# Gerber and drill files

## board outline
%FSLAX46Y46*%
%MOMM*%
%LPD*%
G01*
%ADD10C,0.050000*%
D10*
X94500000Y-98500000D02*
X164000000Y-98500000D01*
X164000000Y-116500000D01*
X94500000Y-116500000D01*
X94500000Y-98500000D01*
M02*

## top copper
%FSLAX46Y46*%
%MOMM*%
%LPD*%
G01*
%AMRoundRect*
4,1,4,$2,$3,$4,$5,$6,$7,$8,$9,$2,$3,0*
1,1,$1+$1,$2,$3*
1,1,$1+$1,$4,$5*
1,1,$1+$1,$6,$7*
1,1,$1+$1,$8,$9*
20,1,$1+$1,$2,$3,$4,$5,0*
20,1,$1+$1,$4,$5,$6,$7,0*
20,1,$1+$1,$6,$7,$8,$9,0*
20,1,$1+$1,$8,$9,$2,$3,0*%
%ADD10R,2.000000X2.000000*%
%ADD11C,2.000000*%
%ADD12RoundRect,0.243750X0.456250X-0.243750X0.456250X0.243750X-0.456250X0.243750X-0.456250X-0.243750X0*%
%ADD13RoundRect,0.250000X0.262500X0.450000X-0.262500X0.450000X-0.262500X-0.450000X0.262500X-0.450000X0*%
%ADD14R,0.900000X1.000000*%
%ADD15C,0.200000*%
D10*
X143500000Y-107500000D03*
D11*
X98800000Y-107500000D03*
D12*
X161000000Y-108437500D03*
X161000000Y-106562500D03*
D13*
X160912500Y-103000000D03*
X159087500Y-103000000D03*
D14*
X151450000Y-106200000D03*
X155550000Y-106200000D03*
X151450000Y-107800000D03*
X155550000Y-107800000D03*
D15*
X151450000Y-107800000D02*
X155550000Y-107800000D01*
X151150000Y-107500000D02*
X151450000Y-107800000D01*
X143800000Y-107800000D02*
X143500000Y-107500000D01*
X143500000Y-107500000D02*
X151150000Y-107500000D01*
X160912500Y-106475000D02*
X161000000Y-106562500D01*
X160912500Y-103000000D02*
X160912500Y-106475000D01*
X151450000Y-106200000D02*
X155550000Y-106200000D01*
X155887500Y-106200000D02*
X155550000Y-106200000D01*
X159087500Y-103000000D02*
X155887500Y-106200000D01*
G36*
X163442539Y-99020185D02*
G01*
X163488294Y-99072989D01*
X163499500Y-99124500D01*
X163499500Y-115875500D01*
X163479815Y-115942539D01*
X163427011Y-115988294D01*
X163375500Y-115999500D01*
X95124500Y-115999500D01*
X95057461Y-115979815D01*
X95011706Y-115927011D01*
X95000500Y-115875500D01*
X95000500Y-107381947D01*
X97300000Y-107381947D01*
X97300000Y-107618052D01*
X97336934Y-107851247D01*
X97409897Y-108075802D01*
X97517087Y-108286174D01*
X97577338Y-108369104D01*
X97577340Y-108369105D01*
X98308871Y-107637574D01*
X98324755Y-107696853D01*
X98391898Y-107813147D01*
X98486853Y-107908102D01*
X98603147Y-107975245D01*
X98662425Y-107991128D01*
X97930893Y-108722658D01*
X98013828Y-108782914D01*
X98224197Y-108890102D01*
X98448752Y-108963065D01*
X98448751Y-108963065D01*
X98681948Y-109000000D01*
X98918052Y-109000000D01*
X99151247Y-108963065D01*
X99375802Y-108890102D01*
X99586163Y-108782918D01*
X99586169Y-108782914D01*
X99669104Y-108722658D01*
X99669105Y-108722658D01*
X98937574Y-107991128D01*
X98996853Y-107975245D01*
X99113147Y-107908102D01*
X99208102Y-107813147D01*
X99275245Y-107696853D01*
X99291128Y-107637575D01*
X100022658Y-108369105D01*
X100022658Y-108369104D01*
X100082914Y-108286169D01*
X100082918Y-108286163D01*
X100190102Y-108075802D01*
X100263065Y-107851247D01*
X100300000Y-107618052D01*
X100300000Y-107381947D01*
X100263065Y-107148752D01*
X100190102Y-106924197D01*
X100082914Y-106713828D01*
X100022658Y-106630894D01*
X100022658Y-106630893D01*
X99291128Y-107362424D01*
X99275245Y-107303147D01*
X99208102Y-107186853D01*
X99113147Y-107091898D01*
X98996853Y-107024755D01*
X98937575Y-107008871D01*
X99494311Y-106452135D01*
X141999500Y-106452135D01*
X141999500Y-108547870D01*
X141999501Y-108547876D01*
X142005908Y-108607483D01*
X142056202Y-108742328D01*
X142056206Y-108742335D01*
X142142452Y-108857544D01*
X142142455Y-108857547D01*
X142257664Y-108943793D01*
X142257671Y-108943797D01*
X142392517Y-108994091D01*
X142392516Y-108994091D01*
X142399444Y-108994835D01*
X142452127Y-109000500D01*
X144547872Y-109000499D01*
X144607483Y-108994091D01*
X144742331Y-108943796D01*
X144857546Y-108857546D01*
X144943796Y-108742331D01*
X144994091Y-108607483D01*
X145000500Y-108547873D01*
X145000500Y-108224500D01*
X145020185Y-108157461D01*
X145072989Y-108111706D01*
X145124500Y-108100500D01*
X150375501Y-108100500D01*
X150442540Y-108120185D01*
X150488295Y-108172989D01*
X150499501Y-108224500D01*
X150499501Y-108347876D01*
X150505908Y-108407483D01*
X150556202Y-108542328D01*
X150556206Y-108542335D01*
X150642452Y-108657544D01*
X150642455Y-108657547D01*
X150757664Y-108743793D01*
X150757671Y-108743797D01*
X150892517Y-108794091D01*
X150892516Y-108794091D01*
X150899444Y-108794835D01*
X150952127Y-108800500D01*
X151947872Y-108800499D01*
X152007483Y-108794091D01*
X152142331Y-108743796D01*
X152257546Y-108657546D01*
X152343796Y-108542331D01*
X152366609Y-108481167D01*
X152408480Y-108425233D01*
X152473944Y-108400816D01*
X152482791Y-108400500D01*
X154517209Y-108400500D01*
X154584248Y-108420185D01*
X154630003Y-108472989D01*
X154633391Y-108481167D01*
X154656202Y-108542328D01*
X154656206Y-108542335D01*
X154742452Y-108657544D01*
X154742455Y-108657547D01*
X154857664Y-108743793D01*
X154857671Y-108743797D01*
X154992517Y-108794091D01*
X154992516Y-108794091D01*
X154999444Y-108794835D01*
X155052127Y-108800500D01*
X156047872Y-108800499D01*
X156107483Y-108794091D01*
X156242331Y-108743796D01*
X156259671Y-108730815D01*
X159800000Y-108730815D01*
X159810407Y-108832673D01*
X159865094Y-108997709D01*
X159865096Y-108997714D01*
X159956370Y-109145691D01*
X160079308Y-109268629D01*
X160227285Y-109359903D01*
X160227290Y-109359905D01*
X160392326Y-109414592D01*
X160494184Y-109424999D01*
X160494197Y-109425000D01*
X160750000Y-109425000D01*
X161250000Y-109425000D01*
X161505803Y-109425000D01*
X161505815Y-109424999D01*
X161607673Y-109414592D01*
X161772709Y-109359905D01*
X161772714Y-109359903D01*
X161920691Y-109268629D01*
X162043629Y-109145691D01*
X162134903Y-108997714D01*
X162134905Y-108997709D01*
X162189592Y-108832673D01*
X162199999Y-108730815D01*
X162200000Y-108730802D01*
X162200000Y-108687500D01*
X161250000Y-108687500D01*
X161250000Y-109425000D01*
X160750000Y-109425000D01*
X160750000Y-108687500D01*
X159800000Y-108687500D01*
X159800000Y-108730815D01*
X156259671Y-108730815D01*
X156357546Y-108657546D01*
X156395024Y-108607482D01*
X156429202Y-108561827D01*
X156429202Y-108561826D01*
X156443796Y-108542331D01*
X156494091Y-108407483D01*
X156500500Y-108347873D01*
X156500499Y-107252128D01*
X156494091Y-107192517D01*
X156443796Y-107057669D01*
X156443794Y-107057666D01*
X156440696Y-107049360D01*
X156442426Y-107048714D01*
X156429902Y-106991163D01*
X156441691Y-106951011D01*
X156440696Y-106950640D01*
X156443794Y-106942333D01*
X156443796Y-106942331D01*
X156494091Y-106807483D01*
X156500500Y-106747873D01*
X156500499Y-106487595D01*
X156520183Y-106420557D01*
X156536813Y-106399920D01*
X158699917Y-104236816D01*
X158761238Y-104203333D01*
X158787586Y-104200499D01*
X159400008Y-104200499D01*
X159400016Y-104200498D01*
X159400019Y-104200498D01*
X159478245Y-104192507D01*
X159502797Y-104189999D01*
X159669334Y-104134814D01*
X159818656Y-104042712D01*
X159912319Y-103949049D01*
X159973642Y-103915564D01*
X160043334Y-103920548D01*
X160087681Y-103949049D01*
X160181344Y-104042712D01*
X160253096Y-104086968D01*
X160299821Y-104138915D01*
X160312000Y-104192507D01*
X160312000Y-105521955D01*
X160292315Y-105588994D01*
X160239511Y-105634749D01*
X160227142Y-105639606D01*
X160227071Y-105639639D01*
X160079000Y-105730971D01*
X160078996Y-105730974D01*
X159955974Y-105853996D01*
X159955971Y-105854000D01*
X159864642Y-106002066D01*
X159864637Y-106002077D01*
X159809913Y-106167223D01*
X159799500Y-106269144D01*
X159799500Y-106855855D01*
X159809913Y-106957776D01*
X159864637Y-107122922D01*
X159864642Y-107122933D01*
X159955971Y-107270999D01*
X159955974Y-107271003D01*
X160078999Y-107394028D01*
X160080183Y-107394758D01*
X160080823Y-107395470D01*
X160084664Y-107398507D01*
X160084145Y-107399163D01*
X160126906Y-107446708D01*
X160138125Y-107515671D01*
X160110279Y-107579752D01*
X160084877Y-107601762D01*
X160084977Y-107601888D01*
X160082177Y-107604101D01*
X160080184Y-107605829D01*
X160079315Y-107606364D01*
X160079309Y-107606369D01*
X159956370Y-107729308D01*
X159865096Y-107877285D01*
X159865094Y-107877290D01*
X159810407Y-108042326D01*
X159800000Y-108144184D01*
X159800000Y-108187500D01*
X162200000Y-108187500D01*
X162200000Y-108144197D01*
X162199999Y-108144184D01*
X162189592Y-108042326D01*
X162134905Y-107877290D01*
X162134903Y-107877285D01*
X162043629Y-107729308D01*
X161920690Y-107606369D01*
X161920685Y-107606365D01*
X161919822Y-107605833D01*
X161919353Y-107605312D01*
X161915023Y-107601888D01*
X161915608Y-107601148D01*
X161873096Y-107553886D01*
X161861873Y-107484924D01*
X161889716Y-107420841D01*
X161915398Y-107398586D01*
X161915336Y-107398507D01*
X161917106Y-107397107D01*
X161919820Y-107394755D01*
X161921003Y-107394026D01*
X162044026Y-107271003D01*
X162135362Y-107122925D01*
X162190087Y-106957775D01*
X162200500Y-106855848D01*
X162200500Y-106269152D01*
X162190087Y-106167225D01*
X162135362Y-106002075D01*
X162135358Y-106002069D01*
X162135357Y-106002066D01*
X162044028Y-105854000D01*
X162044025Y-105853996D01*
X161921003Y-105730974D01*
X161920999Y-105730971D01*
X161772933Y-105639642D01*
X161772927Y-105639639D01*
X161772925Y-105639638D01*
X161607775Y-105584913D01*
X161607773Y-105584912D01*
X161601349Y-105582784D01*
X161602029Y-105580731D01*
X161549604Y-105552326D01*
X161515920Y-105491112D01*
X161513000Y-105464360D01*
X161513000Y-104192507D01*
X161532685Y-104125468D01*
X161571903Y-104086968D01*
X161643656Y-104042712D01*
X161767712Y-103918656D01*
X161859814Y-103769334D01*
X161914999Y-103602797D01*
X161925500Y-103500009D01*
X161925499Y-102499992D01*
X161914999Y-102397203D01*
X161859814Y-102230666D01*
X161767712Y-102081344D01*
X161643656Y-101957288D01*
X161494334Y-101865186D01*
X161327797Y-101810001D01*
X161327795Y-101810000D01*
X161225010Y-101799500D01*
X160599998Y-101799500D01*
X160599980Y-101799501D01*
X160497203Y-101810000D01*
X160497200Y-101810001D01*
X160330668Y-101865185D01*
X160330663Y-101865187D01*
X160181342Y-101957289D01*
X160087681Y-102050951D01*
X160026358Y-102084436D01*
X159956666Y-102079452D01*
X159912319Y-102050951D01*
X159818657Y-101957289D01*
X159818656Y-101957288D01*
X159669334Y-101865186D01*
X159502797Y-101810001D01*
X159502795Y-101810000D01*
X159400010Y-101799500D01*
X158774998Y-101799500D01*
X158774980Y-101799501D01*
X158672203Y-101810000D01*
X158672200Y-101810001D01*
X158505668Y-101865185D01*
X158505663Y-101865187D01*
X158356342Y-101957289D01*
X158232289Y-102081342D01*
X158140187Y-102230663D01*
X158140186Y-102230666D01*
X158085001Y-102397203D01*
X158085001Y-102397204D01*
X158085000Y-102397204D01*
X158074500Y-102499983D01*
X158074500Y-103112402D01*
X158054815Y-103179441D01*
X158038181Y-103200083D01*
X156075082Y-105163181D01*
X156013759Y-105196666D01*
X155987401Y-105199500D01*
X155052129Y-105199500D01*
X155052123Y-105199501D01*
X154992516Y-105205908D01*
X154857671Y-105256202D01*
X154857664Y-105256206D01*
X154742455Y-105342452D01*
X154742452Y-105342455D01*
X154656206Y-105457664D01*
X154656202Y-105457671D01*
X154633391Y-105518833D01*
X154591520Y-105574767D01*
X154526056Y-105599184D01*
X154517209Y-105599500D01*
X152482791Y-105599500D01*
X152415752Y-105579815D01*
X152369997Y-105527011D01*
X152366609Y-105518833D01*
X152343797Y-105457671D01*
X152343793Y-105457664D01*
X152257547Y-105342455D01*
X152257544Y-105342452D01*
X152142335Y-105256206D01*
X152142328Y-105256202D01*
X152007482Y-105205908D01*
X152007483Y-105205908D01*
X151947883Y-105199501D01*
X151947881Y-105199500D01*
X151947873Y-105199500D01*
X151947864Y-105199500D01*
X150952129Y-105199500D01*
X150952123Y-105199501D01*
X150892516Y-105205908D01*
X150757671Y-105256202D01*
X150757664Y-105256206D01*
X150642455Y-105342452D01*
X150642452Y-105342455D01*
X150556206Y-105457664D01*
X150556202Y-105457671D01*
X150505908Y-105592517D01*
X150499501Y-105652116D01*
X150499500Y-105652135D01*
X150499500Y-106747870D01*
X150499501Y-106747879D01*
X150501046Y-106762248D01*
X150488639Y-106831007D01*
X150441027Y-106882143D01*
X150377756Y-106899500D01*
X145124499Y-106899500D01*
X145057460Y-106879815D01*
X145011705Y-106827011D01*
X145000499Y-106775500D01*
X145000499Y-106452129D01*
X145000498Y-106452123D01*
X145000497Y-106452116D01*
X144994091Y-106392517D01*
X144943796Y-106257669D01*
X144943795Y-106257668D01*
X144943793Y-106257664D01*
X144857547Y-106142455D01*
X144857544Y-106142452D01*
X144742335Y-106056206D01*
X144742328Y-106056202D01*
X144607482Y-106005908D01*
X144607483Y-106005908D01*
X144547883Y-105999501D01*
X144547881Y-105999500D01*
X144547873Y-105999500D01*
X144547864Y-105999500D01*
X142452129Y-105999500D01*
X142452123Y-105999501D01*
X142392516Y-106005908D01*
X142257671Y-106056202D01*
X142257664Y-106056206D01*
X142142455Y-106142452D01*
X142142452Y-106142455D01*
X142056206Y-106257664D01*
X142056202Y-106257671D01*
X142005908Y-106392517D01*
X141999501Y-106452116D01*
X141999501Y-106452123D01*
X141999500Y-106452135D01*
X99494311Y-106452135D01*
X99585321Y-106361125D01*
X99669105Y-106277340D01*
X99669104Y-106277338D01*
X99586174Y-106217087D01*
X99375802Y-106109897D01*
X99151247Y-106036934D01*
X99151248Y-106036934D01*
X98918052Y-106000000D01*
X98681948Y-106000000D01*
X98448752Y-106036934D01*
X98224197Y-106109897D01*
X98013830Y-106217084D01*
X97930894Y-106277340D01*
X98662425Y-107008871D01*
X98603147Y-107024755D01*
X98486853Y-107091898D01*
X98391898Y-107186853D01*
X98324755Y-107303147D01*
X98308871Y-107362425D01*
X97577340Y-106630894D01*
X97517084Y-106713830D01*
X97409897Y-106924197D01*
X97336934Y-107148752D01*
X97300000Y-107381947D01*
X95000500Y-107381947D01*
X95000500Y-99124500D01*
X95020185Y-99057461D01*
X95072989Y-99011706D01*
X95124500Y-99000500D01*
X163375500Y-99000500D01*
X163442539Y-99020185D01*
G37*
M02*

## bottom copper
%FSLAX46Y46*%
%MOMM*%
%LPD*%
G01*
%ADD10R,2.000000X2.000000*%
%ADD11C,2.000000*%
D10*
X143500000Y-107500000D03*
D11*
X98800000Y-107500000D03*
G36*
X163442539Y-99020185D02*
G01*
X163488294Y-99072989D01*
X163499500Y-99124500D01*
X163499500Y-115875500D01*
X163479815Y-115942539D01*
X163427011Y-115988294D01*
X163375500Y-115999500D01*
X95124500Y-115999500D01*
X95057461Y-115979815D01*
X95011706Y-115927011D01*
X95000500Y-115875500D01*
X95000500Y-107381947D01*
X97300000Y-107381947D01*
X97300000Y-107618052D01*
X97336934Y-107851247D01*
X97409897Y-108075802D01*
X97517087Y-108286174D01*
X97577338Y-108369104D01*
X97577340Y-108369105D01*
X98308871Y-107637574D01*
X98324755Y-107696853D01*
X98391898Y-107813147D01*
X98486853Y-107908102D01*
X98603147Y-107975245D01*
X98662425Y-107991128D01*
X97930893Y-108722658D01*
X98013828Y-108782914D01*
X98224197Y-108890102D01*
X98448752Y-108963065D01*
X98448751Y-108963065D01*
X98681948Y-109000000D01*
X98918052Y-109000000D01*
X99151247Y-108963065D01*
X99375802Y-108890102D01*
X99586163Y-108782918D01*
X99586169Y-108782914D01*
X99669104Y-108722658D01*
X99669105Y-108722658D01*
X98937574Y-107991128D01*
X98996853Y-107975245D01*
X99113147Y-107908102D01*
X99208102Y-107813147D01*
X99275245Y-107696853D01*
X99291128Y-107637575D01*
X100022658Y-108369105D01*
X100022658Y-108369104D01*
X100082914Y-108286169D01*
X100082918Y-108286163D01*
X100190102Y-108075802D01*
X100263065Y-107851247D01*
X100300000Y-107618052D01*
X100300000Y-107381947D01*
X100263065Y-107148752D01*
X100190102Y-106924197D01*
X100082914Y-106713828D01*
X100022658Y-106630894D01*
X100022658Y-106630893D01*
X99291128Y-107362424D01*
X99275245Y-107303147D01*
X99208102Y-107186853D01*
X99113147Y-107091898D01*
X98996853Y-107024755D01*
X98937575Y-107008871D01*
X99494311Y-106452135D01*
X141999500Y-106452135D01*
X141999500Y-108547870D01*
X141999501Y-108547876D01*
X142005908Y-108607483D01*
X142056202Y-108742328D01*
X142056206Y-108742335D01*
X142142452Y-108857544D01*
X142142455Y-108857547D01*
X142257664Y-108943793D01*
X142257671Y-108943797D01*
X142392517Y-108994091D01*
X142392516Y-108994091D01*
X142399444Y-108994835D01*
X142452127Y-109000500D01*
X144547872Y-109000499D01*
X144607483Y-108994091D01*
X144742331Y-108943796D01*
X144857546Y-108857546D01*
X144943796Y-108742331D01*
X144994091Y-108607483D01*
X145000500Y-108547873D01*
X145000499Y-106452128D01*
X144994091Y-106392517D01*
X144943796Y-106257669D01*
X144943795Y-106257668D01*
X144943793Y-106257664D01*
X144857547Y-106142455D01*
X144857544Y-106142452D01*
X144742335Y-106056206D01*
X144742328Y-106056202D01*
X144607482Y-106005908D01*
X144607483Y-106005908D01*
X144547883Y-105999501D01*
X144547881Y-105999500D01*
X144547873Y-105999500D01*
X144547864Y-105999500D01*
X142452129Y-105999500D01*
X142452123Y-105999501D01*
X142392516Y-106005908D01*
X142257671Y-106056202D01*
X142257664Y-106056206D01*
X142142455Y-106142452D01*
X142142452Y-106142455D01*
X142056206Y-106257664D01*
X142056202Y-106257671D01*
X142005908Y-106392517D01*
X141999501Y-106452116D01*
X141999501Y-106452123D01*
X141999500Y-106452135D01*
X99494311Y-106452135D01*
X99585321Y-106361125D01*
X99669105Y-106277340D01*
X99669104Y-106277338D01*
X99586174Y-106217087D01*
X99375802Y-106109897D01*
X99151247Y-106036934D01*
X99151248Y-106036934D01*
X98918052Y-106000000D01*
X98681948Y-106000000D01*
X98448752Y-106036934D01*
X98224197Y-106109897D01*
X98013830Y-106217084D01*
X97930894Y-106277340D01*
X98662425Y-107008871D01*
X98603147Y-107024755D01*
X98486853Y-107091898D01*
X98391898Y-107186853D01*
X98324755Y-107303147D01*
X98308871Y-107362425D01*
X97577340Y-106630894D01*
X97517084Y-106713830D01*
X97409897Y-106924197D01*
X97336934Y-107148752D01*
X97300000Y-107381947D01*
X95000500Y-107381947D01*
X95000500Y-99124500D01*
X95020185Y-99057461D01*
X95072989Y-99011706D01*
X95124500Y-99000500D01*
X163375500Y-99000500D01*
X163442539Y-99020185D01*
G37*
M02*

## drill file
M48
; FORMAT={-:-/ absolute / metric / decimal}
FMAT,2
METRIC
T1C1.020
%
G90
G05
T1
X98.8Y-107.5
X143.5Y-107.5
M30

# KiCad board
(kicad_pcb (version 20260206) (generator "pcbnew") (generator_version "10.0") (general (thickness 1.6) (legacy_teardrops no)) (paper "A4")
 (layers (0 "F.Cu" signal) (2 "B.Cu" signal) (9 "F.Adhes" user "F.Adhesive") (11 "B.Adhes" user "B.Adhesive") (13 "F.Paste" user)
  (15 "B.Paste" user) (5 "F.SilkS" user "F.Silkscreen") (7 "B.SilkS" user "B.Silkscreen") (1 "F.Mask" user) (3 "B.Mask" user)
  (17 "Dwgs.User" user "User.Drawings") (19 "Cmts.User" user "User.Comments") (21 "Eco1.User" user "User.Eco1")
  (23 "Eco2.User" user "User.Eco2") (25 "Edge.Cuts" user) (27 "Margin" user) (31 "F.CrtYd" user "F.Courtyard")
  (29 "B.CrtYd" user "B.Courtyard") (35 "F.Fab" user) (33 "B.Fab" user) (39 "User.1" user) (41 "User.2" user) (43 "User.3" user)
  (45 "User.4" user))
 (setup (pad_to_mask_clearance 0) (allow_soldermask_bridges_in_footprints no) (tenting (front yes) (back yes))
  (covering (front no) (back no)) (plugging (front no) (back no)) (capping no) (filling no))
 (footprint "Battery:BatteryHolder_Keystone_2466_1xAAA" (layer "F.Cu") (at 143.5 107.5 180)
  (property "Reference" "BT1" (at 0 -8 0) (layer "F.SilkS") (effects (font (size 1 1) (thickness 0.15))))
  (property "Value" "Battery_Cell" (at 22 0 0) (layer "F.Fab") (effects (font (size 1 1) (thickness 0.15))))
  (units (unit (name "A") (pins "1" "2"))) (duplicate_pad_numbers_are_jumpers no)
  (pad "1" thru_hole rect (at 0 0 180) (size 2 2) (drill 1.02) (layers "*.Cu" "*.Mask") (remove_unused_layers no) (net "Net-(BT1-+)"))
  (pad "2" thru_hole circle (at 44.7 0 180) (size 2 2) (drill 1.02) (layers "*.Cu" "*.Mask") (remove_unused_layers no) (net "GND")))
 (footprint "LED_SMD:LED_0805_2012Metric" (layer "F.Cu") (at 161 107.5 90)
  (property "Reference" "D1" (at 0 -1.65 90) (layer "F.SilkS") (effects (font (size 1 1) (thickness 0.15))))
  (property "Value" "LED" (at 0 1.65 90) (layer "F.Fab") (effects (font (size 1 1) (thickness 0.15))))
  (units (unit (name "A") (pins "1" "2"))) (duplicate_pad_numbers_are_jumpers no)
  (pad "1" smd roundrect (at -0.9375 0 90) (size 0.975 1.4) (layers "F.Cu" "F.Mask" "F.Paste") (roundrect_rratio 0.25) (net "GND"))
  (pad "2" smd roundrect (at 0.9375 0 90) (size 0.975 1.4) (layers "F.Cu" "F.Mask" "F.Paste") (roundrect_rratio 0.25) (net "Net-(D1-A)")))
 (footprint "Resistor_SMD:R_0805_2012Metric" (layer "F.Cu") (at 160 103 180)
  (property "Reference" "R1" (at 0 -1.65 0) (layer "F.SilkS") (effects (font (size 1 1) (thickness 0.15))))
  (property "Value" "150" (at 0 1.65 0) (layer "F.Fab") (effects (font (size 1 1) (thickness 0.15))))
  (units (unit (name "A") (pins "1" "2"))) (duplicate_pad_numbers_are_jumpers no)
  (pad "1" smd roundrect (at -0.9125 0 180) (size 1.025 1.4) (layers "F.Cu" "F.Mask" "F.Paste") (roundrect_rratio 0.243902)
   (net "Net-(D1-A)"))
  (pad "2" smd roundrect (at 0.9125 0 180) (size 1.025 1.4) (layers "F.Cu" "F.Mask" "F.Paste") (roundrect_rratio 0.243902)
   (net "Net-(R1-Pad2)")))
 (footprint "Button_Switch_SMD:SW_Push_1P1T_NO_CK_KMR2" (layer "F.Cu") (at 153.5 107)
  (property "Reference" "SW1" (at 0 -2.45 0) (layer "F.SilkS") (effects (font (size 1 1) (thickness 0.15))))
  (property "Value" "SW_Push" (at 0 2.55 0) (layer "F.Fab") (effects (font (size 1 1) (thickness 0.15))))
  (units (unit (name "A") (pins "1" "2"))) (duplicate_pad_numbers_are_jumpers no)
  (pad "1" smd rect (at -2.05 -0.8) (size 0.9 1) (layers "F.Cu" "F.Mask" "F.Paste") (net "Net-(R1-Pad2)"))
  (pad "1" smd rect (at 2.05 -0.8) (size 0.9 1) (layers "F.Cu" "F.Mask" "F.Paste") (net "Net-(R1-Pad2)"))
  (pad "2" smd rect (at -2.05 0.8) (size 0.9 1) (layers "F.Cu" "F.Mask" "F.Paste") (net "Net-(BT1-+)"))
  (pad "2" smd rect (at 2.05 0.8) (size 0.9 1) (layers "F.Cu" "F.Mask" "F.Paste") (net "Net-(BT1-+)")))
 (gr_rect (start 94.5 98.5) (end 164 116.5) (stroke (width 0.05) (type default)) (fill no) (layer "Edge.Cuts"))
 (segment (start 151.45 107.8) (end 155.55 107.8) (width 0.2) (layer "F.Cu") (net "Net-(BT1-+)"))
 (segment (start 151.15 107.5) (end 151.45 107.8) (width 0.2) (layer "F.Cu") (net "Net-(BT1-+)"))
 (segment (start 143.8 107.8) (end 143.5 107.5) (width 0.2) (layer "F.Cu") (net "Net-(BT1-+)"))
 (segment (start 143.5 107.5) (end 151.15 107.5) (width 0.2) (layer "F.Cu") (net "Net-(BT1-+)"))
 (segment (start 160.9125 106.475) (end 161 106.5625) (width 0.2) (layer "F.Cu") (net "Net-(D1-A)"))
 (segment (start 160.9125 103) (end 160.9125 106.475) (width 0.2) (layer "F.Cu") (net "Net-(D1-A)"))
 (segment (start 151.45 106.2) (end 155.55 106.2) (width 0.2) (layer "F.Cu") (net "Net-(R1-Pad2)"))
 (segment (start 155.8875 106.2) (end 155.55 106.2) (width 0.2) (layer "F.Cu") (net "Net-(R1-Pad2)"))
 (segment (start 159.0875 103) (end 155.8875 106.2) (width 0.2) (layer "F.Cu") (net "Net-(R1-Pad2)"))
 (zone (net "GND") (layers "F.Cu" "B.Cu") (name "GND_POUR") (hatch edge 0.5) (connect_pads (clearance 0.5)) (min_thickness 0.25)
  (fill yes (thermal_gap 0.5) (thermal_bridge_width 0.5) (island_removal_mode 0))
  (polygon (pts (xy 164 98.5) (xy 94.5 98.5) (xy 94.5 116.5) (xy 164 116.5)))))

